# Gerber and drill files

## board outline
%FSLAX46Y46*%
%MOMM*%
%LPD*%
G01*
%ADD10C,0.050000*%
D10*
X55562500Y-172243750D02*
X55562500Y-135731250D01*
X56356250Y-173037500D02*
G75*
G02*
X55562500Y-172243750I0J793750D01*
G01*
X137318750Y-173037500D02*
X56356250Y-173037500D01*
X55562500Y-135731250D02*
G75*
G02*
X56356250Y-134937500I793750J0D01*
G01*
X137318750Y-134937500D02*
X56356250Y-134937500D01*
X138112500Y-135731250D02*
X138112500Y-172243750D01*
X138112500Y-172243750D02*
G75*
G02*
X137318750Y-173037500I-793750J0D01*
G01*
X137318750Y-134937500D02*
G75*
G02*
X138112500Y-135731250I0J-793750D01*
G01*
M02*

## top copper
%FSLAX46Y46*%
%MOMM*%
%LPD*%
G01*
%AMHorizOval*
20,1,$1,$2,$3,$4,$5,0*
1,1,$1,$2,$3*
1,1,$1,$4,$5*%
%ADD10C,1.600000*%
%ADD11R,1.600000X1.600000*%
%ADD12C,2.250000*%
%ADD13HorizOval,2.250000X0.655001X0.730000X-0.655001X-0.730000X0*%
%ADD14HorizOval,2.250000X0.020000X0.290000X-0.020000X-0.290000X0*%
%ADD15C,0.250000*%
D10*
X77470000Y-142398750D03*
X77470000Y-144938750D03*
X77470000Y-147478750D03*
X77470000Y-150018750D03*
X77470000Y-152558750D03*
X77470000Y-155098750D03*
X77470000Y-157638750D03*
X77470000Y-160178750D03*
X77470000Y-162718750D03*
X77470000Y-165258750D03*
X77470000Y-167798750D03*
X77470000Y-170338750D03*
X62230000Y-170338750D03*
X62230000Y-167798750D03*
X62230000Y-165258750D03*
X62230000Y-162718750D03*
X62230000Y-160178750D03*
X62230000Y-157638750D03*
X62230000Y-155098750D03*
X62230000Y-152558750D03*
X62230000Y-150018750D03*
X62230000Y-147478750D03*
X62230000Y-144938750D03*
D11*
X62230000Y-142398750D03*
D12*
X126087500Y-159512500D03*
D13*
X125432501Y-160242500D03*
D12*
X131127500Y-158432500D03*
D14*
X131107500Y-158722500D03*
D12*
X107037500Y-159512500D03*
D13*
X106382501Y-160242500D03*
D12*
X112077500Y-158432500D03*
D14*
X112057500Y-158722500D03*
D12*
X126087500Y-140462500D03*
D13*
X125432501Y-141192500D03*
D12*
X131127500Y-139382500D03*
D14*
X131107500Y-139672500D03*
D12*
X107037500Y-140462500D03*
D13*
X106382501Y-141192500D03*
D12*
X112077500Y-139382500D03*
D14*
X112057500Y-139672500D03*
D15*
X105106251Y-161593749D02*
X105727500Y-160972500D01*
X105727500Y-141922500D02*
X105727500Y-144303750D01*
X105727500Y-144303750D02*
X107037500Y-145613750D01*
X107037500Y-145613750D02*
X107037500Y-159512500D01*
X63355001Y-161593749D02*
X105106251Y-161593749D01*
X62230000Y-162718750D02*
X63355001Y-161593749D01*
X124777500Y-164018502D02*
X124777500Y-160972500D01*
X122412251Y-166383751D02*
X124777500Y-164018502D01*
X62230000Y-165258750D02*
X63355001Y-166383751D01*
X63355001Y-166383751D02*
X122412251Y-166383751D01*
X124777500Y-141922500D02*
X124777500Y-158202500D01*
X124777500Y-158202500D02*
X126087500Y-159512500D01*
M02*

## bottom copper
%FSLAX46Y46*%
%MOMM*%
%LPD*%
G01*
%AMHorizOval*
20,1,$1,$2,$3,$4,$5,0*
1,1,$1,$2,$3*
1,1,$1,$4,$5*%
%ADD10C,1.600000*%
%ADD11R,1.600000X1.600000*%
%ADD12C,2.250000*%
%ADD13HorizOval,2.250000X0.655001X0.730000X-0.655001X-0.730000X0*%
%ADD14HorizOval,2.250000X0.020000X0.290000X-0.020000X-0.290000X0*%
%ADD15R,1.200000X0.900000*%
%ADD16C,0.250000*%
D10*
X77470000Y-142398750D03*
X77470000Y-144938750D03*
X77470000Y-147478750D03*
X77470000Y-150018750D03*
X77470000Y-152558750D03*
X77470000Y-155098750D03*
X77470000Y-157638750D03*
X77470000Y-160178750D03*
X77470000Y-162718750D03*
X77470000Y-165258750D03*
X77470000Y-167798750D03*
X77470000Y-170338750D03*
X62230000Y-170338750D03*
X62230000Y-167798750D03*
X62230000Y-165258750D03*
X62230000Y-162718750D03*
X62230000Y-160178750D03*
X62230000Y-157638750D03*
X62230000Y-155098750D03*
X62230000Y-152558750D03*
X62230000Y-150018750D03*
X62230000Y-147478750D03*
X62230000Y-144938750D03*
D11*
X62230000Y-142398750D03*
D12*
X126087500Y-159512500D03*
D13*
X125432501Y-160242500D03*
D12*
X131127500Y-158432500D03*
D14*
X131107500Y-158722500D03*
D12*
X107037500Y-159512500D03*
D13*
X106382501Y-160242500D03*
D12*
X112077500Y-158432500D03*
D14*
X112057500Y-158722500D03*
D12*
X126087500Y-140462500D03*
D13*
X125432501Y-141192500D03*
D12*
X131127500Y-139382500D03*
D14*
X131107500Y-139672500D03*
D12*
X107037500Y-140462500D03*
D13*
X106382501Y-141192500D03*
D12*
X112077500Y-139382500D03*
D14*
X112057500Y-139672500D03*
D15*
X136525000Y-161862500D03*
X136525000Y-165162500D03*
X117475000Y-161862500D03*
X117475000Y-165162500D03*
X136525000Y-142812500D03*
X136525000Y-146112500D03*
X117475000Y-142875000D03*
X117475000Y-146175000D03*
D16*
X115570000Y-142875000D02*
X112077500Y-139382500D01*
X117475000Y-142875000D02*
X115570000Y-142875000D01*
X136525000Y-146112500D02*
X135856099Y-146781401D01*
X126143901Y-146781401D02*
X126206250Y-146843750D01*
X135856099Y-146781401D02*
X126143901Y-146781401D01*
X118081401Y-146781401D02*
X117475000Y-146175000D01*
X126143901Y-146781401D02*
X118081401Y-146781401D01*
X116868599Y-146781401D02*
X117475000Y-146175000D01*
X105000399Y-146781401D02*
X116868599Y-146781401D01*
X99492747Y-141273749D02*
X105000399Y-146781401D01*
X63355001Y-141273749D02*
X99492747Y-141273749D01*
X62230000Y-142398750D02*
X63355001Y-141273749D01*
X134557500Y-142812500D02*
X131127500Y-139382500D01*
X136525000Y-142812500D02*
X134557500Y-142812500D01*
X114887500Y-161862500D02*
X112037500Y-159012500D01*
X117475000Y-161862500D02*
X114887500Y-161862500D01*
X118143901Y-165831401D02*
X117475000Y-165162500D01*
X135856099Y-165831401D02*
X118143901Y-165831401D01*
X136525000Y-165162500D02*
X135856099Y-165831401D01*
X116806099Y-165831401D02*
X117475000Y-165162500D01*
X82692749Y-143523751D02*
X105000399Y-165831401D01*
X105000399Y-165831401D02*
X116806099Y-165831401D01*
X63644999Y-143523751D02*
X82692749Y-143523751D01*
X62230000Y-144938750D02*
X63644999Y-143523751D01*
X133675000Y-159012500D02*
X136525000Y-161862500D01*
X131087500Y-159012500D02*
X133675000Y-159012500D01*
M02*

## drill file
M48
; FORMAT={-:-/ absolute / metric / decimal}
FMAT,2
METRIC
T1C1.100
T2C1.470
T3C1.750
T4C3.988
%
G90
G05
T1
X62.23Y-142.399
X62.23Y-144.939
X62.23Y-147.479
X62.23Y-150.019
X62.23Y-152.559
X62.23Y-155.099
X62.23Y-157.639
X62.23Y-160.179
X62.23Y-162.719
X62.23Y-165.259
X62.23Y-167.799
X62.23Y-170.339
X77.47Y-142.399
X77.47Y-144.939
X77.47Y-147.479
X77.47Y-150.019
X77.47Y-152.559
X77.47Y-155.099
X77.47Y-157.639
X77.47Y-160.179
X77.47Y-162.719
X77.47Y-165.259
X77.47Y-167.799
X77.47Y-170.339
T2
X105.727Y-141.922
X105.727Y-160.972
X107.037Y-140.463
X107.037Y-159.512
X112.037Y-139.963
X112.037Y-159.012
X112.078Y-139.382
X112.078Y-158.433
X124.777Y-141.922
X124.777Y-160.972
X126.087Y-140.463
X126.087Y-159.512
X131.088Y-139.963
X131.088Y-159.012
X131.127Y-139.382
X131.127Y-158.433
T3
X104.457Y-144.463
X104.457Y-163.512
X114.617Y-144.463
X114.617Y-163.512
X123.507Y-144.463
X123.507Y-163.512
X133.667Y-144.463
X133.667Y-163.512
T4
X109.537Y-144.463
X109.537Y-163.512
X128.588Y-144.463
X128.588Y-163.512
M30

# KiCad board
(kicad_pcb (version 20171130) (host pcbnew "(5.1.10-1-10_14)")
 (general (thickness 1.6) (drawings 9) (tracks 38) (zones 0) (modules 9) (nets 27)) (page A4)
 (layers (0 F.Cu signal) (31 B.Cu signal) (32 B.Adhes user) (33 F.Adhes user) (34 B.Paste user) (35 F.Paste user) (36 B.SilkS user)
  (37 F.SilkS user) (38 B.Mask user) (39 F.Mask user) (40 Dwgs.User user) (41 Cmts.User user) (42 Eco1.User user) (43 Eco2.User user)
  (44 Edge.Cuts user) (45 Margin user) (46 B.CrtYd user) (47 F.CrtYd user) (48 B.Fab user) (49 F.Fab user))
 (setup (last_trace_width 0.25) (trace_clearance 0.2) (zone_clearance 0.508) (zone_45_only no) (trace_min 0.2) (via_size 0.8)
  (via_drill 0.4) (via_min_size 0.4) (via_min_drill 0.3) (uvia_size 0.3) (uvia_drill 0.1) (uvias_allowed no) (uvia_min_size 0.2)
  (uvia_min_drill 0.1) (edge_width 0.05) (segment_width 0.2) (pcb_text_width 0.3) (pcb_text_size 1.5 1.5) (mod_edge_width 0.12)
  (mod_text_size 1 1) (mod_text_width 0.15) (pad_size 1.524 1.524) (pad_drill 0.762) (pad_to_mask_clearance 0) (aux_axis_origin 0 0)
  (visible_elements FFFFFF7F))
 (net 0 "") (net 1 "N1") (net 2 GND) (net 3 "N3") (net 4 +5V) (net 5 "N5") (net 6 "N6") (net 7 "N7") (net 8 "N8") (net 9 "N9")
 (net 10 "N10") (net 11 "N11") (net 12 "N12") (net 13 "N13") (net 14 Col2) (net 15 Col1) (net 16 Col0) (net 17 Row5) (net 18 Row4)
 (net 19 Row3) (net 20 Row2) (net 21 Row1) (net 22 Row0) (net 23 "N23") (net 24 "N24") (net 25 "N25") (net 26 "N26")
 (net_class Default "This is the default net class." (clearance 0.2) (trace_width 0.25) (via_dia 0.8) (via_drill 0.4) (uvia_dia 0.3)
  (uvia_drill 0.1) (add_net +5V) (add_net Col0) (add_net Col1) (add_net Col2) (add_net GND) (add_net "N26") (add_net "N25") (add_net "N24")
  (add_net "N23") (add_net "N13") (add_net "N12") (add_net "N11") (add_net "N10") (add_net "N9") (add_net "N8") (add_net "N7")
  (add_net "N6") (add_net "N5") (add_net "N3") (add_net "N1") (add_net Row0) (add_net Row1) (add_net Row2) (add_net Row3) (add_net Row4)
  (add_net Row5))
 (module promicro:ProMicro (layer F.Cu) (at 69.85 156.36875 270)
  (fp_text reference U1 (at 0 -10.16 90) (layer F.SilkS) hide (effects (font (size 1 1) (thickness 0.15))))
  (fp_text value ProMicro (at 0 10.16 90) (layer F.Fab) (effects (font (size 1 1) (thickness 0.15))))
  (pad 24 thru_hole circle (at -13.97 -7.62 270) (size 1.6 1.6) (drill 1.1) (layers *.Cu *.Mask F.SilkS) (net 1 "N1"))
  (pad 23 thru_hole circle (at -11.43 -7.62 270) (size 1.6 1.6) (drill 1.1) (layers *.Cu *.Mask F.SilkS) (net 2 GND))
  (pad 22 thru_hole circle (at -8.89 -7.62 270) (size 1.6 1.6) (drill 1.1) (layers *.Cu *.Mask F.SilkS) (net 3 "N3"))
  (pad 21 thru_hole circle (at -6.35 -7.62 270) (size 1.6 1.6) (drill 1.1) (layers *.Cu *.Mask F.SilkS) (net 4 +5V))
  (pad 20 thru_hole circle (at -3.81 -7.62 270) (size 1.6 1.6) (drill 1.1) (layers *.Cu *.Mask F.SilkS) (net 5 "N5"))
  (pad 19 thru_hole circle (at -1.27 -7.62 270) (size 1.6 1.6) (drill 1.1) (layers *.Cu *.Mask F.SilkS) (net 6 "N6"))
  (pad 18 thru_hole circle (at 1.27 -7.62 270) (size 1.6 1.6) (drill 1.1) (layers *.Cu *.Mask F.SilkS) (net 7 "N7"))
  (pad 17 thru_hole circle (at 3.81 -7.62 270) (size 1.6 1.6) (drill 1.1) (layers *.Cu *.Mask F.SilkS) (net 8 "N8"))
  (pad 16 thru_hole circle (at 6.35 -7.62 270) (size 1.6 1.6) (drill 1.1) (layers *.Cu *.Mask F.SilkS) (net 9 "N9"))
  (pad 15 thru_hole circle (at 8.89 -7.62 270) (size 1.6 1.6) (drill 1.1) (layers *.Cu *.Mask F.SilkS) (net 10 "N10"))
  (pad 14 thru_hole circle (at 11.43 -7.62 270) (size 1.6 1.6) (drill 1.1) (layers *.Cu *.Mask F.SilkS) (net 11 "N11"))
  (pad 13 thru_hole circle (at 13.97 -7.62 270) (size 1.6 1.6) (drill 1.1) (layers *.Cu *.Mask F.SilkS) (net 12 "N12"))
  (pad 12 thru_hole circle (at 13.97 7.62 270) (size 1.6 1.6) (drill 1.1) (layers *.Cu *.Mask F.SilkS) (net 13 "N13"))
  (pad 11 thru_hole circle (at 11.43 7.62 270) (size 1.6 1.6) (drill 1.1) (layers *.Cu *.Mask F.SilkS) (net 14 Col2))
  (pad 10 thru_hole circle (at 8.89 7.62 270) (size 1.6 1.6) (drill 1.1) (layers *.Cu *.Mask F.SilkS) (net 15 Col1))
  (pad 9 thru_hole circle (at 6.35 7.62 270) (size 1.6 1.6) (drill 1.1) (layers *.Cu *.Mask F.SilkS) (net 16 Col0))
  (pad 8 thru_hole circle (at 3.81 7.62 270) (size 1.6 1.6) (drill 1.1) (layers *.Cu *.Mask F.SilkS) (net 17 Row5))
  (pad 7 thru_hole circle (at 1.27 7.62 270) (size 1.6 1.6) (drill 1.1) (layers *.Cu *.Mask F.SilkS) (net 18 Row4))
  (pad 6 thru_hole circle (at -1.27 7.62 270) (size 1.6 1.6) (drill 1.1) (layers *.Cu *.Mask F.SilkS) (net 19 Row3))
  (pad 5 thru_hole circle (at -3.81 7.62 270) (size 1.6 1.6) (drill 1.1) (layers *.Cu *.Mask F.SilkS) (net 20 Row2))
  (pad 4 thru_hole circle (at -6.35 7.62 270) (size 1.6 1.6) (drill 1.1) (layers *.Cu *.Mask F.SilkS) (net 2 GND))
  (pad 3 thru_hole circle (at -8.89 7.62 270) (size 1.6 1.6) (drill 1.1) (layers *.Cu *.Mask F.SilkS) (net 2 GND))
  (pad 2 thru_hole circle (at -11.43 7.62 270) (size 1.6 1.6) (drill 1.1) (layers *.Cu *.Mask F.SilkS) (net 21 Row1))
  (pad 1 thru_hole rect (at -13.97 7.62 270) (size 1.6 1.6) (drill 1.1) (layers *.Cu *.Mask F.SilkS) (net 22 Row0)))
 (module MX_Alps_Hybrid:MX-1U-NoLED (layer F.Cu) (at 128.5875 163.5125)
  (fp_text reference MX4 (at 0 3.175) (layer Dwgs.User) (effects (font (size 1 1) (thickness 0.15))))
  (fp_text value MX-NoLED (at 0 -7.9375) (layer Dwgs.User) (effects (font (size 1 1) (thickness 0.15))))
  (pad "" np_thru_hole circle (at 5.08 0 48.0996) (size 1.75 1.75) (drill 1.75) (layers *.Cu *.Mask))
  (pad "" np_thru_hole circle (at -5.08 0 48.0996) (size 1.75 1.75) (drill 1.75) (layers *.Cu *.Mask))
  (pad 1 thru_hole circle (at -2.5 -4) (size 2.25 2.25) (drill 1.47) (layers *.Cu B.Mask) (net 15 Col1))
  (pad "" np_thru_hole circle (at 0 0) (size 3.9878 3.9878) (drill 3.9878) (layers *.Cu *.Mask))
  (pad 1 thru_hole oval (at -3.81 -2.54 48.0996) (size 4.211556 2.25) (drill 1.47 (offset 0.980778 0)) (layers *.Cu B.Mask) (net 15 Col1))
  (pad 2 thru_hole circle (at 2.54 -5.08) (size 2.25 2.25) (drill 1.47) (layers *.Cu B.Mask) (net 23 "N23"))
  (pad 2 thru_hole oval (at 2.5 -4.5 86.0548) (size 2.831378 2.25) (drill 1.47 (offset 0.290689 0)) (layers *.Cu B.Mask) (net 23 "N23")))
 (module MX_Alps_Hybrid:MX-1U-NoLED (layer F.Cu) (at 109.5375 163.5125)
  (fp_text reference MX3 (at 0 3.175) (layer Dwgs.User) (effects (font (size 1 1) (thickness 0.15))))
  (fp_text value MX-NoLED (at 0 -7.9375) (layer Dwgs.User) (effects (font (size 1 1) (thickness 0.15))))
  (pad "" np_thru_hole circle (at 5.08 0 48.0996) (size 1.75 1.75) (drill 1.75) (layers *.Cu *.Mask))
  (pad "" np_thru_hole circle (at -5.08 0 48.0996) (size 1.75 1.75) (drill 1.75) (layers *.Cu *.Mask))
  (pad 1 thru_hole circle (at -2.5 -4) (size 2.25 2.25) (drill 1.47) (layers *.Cu B.Mask) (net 16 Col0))
  (pad "" np_thru_hole circle (at 0 0) (size 3.9878 3.9878) (drill 3.9878) (layers *.Cu *.Mask))
  (pad 1 thru_hole oval (at -3.81 -2.54 48.0996) (size 4.211556 2.25) (drill 1.47 (offset 0.980778 0)) (layers *.Cu B.Mask) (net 16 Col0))
  (pad 2 thru_hole circle (at 2.54 -5.08) (size 2.25 2.25) (drill 1.47) (layers *.Cu B.Mask) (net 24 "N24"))
  (pad 2 thru_hole oval (at 2.5 -4.5 86.0548) (size 2.831378 2.25) (drill 1.47 (offset 0.290689 0)) (layers *.Cu B.Mask) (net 24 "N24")))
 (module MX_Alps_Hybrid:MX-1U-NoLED (layer F.Cu) (at 128.5875 144.4625)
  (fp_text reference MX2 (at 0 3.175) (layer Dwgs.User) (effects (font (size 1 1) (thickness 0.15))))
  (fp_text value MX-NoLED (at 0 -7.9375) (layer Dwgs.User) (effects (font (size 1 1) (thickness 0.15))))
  (pad "" np_thru_hole circle (at 5.08 0 48.0996) (size 1.75 1.75) (drill 1.75) (layers *.Cu *.Mask))
  (pad "" np_thru_hole circle (at -5.08 0 48.0996) (size 1.75 1.75) (drill 1.75) (layers *.Cu *.Mask))
  (pad 1 thru_hole circle (at -2.5 -4) (size 2.25 2.25) (drill 1.47) (layers *.Cu B.Mask) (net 15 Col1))
  (pad "" np_thru_hole circle (at 0 0) (size 3.9878 3.9878) (drill 3.9878) (layers *.Cu *.Mask))
  (pad 1 thru_hole oval (at -3.81 -2.54 48.0996) (size 4.211556 2.25) (drill 1.47 (offset 0.980778 0)) (layers *.Cu B.Mask) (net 15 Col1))
  (pad 2 thru_hole circle (at 2.54 -5.08) (size 2.25 2.25) (drill 1.47) (layers *.Cu B.Mask) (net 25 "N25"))
  (pad 2 thru_hole oval (at 2.5 -4.5 86.0548) (size 2.831378 2.25) (drill 1.47 (offset 0.290689 0)) (layers *.Cu B.Mask) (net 25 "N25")))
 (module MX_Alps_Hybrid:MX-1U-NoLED (layer F.Cu) (at 109.5375 144.4625)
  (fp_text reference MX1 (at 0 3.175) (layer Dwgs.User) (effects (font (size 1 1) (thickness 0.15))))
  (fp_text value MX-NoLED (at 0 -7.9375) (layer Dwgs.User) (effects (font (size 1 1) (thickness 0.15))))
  (pad "" np_thru_hole circle (at 5.08 0 48.0996) (size 1.75 1.75) (drill 1.75) (layers *.Cu *.Mask))
  (pad "" np_thru_hole circle (at -5.08 0 48.0996) (size 1.75 1.75) (drill 1.75) (layers *.Cu *.Mask))
  (pad 1 thru_hole circle (at -2.5 -4) (size 2.25 2.25) (drill 1.47) (layers *.Cu B.Mask) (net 16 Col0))
  (pad "" np_thru_hole circle (at 0 0) (size 3.9878 3.9878) (drill 3.9878) (layers *.Cu *.Mask))
  (pad 1 thru_hole oval (at -3.81 -2.54 48.0996) (size 4.211556 2.25) (drill 1.47 (offset 0.980778 0)) (layers *.Cu B.Mask) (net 16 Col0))
  (pad 2 thru_hole circle (at 2.54 -5.08) (size 2.25 2.25) (drill 1.47) (layers *.Cu B.Mask) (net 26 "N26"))
  (pad 2 thru_hole oval (at 2.5 -4.5 86.0548) (size 2.831378 2.25) (drill 1.47 (offset 0.290689 0)) (layers *.Cu B.Mask) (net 26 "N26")))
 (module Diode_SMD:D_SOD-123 (layer B.Cu) (at 136.525 163.5125 90)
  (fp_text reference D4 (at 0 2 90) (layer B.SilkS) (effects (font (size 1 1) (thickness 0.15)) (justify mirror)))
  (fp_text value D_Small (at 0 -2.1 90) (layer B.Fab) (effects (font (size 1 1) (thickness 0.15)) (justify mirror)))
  (pad 2 smd rect (at 1.65 0 90) (size 0.9 1.2) (layers B.Cu B.Paste B.Mask) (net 23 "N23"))
  (pad 1 smd rect (at -1.65 0 90) (size 0.9 1.2) (layers B.Cu B.Paste B.Mask) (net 21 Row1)))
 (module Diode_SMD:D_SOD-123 (layer B.Cu) (at 117.475 163.5125 90)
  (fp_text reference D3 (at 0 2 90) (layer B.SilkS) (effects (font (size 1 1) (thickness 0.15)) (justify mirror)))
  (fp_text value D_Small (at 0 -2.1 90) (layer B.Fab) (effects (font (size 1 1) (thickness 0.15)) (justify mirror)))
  (pad 2 smd rect (at 1.65 0 90) (size 0.9 1.2) (layers B.Cu B.Paste B.Mask) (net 24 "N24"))
  (pad 1 smd rect (at -1.65 0 90) (size 0.9 1.2) (layers B.Cu B.Paste B.Mask) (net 21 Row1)))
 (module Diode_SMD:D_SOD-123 (layer B.Cu) (at 136.525 144.4625 90)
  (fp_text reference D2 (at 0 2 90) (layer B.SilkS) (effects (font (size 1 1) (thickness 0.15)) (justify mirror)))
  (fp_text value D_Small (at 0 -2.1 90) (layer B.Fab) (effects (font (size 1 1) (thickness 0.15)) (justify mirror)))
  (pad 2 smd rect (at 1.65 0 90) (size 0.9 1.2) (layers B.Cu B.Paste B.Mask) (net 25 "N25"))
  (pad 1 smd rect (at -1.65 0 90) (size 0.9 1.2) (layers B.Cu B.Paste B.Mask) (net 22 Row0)))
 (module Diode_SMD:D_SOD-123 (layer B.Cu) (at 117.475 144.525 90)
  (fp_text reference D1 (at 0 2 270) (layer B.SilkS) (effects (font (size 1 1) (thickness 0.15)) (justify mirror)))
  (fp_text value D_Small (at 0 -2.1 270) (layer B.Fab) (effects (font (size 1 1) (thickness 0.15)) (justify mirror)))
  (pad 2 smd rect (at 1.65 0 90) (size 0.9 1.2) (layers B.Cu B.Paste B.Mask) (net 26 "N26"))
  (pad 1 smd rect (at -1.65 0 90) (size 0.9 1.2) (layers B.Cu B.Paste B.Mask) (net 22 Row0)))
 (gr_line (start 55.5625 172.24375) (end 55.5625 135.73125) (layer Edge.Cuts) (width 0.05))
 (gr_arc (start 56.35625 172.24375) (end 55.5625 172.24375) (angle -90) (layer Edge.Cuts) (width 0.05))
 (gr_line (start 137.31875 173.0375) (end 56.35625 173.0375) (layer Edge.Cuts) (width 0.05))
 (gr_arc (start 56.35625 135.73125) (end 56.35625 134.9375) (angle -90) (layer Edge.Cuts) (width 0.05))
 (gr_line (start 137.31875 134.9375) (end 56.35625 134.9375) (layer Edge.Cuts) (width 0.05))
 (gr_line (start 138.1125 135.73125) (end 138.1125 172.24375) (layer Edge.Cuts) (width 0.05))
 (gr_arc (start 137.31875 172.24375) (end 137.31875 173.0375) (angle -90) (layer Edge.Cuts) (width 0.05))
 (gr_arc (start 137.31875 135.73125) (end 138.1125 135.73125) (angle -90) (layer Edge.Cuts) (width 0.05))
 (segment (start 115.57 142.875) (end 112.0775 139.3825) (width 0.25) (layer B.Cu) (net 26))
 (segment (start 117.475 142.875) (end 115.57 142.875) (width 0.25) (layer B.Cu) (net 26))
 (segment (start 136.525 146.1125) (end 135.856099 146.781401) (width 0.25) (layer B.Cu) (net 22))
 (segment (start 126.143901 146.781401) (end 126.20625 146.84375) (width 0.25) (layer B.Cu) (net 22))
 (segment (start 135.856099 146.781401) (end 126.143901 146.781401) (width 0.25) (layer B.Cu) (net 22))
 (segment (start 118.081401 146.781401) (end 117.475 146.175) (width 0.25) (layer B.Cu) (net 22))
 (segment (start 126.143901 146.781401) (end 118.081401 146.781401) (width 0.25) (layer B.Cu) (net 22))
 (segment (start 116.868599 146.781401) (end 117.475 146.175) (width 0.25) (layer B.Cu) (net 22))
 (segment (start 105.000399 146.781401) (end 116.868599 146.781401) (width 0.25) (layer B.Cu) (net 22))
 (segment (start 99.492747 141.273749) (end 105.000399 146.781401) (width 0.25) (layer B.Cu) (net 22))
 (segment (start 63.355001 141.273749) (end 99.492747 141.273749) (width 0.25) (layer B.Cu) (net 22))
 (segment (start 62.23 142.39875) (end 63.355001 141.273749) (width 0.25) (layer B.Cu) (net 22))
 (segment (start 134.5575 142.8125) (end 131.1275 139.3825) (width 0.25) (layer B.Cu) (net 25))
 (segment (start 136.525 142.8125) (end 134.5575 142.8125) (width 0.25) (layer B.Cu) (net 25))
 (segment (start 114.8875 161.8625) (end 112.0375 159.0125) (width 0.25) (layer B.Cu) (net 24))
 (segment (start 117.475 161.8625) (end 114.8875 161.8625) (width 0.25) (layer B.Cu) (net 24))
 (segment (start 118.143901 165.831401) (end 117.475 165.1625) (width 0.25) (layer B.Cu) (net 21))
 (segment (start 135.856099 165.831401) (end 118.143901 165.831401) (width 0.25) (layer B.Cu) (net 21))
 (segment (start 136.525 165.1625) (end 135.856099 165.831401) (width 0.25) (layer B.Cu) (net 21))
 (segment (start 116.806099 165.831401) (end 117.475 165.1625) (width 0.25) (layer B.Cu) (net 21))
 (segment (start 82.692749 143.523751) (end 105.000399 165.831401) (width 0.25) (layer B.Cu) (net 21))
 (segment (start 105.000399 165.831401) (end 116.806099 165.831401) (width 0.25) (layer B.Cu) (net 21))
 (segment (start 63.644999 143.523751) (end 82.692749 143.523751) (width 0.25) (layer B.Cu) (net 21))
 (segment (start 62.23 144.93875) (end 63.644999 143.523751) (width 0.25) (layer B.Cu) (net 21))
 (segment (start 133.675 159.0125) (end 136.525 161.8625) (width 0.25) (layer B.Cu) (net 23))
 (segment (start 131.0875 159.0125) (end 133.675 159.0125) (width 0.25) (layer B.Cu) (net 23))
 (segment (start 105.106251 161.593749) (end 105.7275 160.9725) (width 0.25) (layer F.Cu) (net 16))
 (segment (start 105.7275 141.9225) (end 105.7275 144.30375) (width 0.25) (layer F.Cu) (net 16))
 (segment (start 105.7275 144.30375) (end 107.0375 145.61375) (width 0.25) (layer F.Cu) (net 16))
 (segment (start 107.0375 145.61375) (end 107.0375 159.5125) (width 0.25) (layer F.Cu) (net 16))
 (segment (start 63.355001 161.593749) (end 105.106251 161.593749) (width 0.25) (layer F.Cu) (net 16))
 (segment (start 62.23 162.71875) (end 63.355001 161.593749) (width 0.25) (layer F.Cu) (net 16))
 (segment (start 124.7775 164.018502) (end 124.7775 160.9725) (width 0.25) (layer F.Cu) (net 15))
 (segment (start 122.412251 166.383751) (end 124.7775 164.018502) (width 0.25) (layer F.Cu) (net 15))
 (segment (start 62.23 165.25875) (end 63.355001 166.383751) (width 0.25) (layer F.Cu) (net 15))
 (segment (start 63.355001 166.383751) (end 122.412251 166.383751) (width 0.25) (layer F.Cu) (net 15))
 (segment (start 124.7775 141.9225) (end 124.7775 158.2025) (width 0.25) (layer F.Cu) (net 15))
 (segment (start 124.7775 158.2025) (end 126.0875 159.5125) (width 0.25) (layer F.Cu) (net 15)))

